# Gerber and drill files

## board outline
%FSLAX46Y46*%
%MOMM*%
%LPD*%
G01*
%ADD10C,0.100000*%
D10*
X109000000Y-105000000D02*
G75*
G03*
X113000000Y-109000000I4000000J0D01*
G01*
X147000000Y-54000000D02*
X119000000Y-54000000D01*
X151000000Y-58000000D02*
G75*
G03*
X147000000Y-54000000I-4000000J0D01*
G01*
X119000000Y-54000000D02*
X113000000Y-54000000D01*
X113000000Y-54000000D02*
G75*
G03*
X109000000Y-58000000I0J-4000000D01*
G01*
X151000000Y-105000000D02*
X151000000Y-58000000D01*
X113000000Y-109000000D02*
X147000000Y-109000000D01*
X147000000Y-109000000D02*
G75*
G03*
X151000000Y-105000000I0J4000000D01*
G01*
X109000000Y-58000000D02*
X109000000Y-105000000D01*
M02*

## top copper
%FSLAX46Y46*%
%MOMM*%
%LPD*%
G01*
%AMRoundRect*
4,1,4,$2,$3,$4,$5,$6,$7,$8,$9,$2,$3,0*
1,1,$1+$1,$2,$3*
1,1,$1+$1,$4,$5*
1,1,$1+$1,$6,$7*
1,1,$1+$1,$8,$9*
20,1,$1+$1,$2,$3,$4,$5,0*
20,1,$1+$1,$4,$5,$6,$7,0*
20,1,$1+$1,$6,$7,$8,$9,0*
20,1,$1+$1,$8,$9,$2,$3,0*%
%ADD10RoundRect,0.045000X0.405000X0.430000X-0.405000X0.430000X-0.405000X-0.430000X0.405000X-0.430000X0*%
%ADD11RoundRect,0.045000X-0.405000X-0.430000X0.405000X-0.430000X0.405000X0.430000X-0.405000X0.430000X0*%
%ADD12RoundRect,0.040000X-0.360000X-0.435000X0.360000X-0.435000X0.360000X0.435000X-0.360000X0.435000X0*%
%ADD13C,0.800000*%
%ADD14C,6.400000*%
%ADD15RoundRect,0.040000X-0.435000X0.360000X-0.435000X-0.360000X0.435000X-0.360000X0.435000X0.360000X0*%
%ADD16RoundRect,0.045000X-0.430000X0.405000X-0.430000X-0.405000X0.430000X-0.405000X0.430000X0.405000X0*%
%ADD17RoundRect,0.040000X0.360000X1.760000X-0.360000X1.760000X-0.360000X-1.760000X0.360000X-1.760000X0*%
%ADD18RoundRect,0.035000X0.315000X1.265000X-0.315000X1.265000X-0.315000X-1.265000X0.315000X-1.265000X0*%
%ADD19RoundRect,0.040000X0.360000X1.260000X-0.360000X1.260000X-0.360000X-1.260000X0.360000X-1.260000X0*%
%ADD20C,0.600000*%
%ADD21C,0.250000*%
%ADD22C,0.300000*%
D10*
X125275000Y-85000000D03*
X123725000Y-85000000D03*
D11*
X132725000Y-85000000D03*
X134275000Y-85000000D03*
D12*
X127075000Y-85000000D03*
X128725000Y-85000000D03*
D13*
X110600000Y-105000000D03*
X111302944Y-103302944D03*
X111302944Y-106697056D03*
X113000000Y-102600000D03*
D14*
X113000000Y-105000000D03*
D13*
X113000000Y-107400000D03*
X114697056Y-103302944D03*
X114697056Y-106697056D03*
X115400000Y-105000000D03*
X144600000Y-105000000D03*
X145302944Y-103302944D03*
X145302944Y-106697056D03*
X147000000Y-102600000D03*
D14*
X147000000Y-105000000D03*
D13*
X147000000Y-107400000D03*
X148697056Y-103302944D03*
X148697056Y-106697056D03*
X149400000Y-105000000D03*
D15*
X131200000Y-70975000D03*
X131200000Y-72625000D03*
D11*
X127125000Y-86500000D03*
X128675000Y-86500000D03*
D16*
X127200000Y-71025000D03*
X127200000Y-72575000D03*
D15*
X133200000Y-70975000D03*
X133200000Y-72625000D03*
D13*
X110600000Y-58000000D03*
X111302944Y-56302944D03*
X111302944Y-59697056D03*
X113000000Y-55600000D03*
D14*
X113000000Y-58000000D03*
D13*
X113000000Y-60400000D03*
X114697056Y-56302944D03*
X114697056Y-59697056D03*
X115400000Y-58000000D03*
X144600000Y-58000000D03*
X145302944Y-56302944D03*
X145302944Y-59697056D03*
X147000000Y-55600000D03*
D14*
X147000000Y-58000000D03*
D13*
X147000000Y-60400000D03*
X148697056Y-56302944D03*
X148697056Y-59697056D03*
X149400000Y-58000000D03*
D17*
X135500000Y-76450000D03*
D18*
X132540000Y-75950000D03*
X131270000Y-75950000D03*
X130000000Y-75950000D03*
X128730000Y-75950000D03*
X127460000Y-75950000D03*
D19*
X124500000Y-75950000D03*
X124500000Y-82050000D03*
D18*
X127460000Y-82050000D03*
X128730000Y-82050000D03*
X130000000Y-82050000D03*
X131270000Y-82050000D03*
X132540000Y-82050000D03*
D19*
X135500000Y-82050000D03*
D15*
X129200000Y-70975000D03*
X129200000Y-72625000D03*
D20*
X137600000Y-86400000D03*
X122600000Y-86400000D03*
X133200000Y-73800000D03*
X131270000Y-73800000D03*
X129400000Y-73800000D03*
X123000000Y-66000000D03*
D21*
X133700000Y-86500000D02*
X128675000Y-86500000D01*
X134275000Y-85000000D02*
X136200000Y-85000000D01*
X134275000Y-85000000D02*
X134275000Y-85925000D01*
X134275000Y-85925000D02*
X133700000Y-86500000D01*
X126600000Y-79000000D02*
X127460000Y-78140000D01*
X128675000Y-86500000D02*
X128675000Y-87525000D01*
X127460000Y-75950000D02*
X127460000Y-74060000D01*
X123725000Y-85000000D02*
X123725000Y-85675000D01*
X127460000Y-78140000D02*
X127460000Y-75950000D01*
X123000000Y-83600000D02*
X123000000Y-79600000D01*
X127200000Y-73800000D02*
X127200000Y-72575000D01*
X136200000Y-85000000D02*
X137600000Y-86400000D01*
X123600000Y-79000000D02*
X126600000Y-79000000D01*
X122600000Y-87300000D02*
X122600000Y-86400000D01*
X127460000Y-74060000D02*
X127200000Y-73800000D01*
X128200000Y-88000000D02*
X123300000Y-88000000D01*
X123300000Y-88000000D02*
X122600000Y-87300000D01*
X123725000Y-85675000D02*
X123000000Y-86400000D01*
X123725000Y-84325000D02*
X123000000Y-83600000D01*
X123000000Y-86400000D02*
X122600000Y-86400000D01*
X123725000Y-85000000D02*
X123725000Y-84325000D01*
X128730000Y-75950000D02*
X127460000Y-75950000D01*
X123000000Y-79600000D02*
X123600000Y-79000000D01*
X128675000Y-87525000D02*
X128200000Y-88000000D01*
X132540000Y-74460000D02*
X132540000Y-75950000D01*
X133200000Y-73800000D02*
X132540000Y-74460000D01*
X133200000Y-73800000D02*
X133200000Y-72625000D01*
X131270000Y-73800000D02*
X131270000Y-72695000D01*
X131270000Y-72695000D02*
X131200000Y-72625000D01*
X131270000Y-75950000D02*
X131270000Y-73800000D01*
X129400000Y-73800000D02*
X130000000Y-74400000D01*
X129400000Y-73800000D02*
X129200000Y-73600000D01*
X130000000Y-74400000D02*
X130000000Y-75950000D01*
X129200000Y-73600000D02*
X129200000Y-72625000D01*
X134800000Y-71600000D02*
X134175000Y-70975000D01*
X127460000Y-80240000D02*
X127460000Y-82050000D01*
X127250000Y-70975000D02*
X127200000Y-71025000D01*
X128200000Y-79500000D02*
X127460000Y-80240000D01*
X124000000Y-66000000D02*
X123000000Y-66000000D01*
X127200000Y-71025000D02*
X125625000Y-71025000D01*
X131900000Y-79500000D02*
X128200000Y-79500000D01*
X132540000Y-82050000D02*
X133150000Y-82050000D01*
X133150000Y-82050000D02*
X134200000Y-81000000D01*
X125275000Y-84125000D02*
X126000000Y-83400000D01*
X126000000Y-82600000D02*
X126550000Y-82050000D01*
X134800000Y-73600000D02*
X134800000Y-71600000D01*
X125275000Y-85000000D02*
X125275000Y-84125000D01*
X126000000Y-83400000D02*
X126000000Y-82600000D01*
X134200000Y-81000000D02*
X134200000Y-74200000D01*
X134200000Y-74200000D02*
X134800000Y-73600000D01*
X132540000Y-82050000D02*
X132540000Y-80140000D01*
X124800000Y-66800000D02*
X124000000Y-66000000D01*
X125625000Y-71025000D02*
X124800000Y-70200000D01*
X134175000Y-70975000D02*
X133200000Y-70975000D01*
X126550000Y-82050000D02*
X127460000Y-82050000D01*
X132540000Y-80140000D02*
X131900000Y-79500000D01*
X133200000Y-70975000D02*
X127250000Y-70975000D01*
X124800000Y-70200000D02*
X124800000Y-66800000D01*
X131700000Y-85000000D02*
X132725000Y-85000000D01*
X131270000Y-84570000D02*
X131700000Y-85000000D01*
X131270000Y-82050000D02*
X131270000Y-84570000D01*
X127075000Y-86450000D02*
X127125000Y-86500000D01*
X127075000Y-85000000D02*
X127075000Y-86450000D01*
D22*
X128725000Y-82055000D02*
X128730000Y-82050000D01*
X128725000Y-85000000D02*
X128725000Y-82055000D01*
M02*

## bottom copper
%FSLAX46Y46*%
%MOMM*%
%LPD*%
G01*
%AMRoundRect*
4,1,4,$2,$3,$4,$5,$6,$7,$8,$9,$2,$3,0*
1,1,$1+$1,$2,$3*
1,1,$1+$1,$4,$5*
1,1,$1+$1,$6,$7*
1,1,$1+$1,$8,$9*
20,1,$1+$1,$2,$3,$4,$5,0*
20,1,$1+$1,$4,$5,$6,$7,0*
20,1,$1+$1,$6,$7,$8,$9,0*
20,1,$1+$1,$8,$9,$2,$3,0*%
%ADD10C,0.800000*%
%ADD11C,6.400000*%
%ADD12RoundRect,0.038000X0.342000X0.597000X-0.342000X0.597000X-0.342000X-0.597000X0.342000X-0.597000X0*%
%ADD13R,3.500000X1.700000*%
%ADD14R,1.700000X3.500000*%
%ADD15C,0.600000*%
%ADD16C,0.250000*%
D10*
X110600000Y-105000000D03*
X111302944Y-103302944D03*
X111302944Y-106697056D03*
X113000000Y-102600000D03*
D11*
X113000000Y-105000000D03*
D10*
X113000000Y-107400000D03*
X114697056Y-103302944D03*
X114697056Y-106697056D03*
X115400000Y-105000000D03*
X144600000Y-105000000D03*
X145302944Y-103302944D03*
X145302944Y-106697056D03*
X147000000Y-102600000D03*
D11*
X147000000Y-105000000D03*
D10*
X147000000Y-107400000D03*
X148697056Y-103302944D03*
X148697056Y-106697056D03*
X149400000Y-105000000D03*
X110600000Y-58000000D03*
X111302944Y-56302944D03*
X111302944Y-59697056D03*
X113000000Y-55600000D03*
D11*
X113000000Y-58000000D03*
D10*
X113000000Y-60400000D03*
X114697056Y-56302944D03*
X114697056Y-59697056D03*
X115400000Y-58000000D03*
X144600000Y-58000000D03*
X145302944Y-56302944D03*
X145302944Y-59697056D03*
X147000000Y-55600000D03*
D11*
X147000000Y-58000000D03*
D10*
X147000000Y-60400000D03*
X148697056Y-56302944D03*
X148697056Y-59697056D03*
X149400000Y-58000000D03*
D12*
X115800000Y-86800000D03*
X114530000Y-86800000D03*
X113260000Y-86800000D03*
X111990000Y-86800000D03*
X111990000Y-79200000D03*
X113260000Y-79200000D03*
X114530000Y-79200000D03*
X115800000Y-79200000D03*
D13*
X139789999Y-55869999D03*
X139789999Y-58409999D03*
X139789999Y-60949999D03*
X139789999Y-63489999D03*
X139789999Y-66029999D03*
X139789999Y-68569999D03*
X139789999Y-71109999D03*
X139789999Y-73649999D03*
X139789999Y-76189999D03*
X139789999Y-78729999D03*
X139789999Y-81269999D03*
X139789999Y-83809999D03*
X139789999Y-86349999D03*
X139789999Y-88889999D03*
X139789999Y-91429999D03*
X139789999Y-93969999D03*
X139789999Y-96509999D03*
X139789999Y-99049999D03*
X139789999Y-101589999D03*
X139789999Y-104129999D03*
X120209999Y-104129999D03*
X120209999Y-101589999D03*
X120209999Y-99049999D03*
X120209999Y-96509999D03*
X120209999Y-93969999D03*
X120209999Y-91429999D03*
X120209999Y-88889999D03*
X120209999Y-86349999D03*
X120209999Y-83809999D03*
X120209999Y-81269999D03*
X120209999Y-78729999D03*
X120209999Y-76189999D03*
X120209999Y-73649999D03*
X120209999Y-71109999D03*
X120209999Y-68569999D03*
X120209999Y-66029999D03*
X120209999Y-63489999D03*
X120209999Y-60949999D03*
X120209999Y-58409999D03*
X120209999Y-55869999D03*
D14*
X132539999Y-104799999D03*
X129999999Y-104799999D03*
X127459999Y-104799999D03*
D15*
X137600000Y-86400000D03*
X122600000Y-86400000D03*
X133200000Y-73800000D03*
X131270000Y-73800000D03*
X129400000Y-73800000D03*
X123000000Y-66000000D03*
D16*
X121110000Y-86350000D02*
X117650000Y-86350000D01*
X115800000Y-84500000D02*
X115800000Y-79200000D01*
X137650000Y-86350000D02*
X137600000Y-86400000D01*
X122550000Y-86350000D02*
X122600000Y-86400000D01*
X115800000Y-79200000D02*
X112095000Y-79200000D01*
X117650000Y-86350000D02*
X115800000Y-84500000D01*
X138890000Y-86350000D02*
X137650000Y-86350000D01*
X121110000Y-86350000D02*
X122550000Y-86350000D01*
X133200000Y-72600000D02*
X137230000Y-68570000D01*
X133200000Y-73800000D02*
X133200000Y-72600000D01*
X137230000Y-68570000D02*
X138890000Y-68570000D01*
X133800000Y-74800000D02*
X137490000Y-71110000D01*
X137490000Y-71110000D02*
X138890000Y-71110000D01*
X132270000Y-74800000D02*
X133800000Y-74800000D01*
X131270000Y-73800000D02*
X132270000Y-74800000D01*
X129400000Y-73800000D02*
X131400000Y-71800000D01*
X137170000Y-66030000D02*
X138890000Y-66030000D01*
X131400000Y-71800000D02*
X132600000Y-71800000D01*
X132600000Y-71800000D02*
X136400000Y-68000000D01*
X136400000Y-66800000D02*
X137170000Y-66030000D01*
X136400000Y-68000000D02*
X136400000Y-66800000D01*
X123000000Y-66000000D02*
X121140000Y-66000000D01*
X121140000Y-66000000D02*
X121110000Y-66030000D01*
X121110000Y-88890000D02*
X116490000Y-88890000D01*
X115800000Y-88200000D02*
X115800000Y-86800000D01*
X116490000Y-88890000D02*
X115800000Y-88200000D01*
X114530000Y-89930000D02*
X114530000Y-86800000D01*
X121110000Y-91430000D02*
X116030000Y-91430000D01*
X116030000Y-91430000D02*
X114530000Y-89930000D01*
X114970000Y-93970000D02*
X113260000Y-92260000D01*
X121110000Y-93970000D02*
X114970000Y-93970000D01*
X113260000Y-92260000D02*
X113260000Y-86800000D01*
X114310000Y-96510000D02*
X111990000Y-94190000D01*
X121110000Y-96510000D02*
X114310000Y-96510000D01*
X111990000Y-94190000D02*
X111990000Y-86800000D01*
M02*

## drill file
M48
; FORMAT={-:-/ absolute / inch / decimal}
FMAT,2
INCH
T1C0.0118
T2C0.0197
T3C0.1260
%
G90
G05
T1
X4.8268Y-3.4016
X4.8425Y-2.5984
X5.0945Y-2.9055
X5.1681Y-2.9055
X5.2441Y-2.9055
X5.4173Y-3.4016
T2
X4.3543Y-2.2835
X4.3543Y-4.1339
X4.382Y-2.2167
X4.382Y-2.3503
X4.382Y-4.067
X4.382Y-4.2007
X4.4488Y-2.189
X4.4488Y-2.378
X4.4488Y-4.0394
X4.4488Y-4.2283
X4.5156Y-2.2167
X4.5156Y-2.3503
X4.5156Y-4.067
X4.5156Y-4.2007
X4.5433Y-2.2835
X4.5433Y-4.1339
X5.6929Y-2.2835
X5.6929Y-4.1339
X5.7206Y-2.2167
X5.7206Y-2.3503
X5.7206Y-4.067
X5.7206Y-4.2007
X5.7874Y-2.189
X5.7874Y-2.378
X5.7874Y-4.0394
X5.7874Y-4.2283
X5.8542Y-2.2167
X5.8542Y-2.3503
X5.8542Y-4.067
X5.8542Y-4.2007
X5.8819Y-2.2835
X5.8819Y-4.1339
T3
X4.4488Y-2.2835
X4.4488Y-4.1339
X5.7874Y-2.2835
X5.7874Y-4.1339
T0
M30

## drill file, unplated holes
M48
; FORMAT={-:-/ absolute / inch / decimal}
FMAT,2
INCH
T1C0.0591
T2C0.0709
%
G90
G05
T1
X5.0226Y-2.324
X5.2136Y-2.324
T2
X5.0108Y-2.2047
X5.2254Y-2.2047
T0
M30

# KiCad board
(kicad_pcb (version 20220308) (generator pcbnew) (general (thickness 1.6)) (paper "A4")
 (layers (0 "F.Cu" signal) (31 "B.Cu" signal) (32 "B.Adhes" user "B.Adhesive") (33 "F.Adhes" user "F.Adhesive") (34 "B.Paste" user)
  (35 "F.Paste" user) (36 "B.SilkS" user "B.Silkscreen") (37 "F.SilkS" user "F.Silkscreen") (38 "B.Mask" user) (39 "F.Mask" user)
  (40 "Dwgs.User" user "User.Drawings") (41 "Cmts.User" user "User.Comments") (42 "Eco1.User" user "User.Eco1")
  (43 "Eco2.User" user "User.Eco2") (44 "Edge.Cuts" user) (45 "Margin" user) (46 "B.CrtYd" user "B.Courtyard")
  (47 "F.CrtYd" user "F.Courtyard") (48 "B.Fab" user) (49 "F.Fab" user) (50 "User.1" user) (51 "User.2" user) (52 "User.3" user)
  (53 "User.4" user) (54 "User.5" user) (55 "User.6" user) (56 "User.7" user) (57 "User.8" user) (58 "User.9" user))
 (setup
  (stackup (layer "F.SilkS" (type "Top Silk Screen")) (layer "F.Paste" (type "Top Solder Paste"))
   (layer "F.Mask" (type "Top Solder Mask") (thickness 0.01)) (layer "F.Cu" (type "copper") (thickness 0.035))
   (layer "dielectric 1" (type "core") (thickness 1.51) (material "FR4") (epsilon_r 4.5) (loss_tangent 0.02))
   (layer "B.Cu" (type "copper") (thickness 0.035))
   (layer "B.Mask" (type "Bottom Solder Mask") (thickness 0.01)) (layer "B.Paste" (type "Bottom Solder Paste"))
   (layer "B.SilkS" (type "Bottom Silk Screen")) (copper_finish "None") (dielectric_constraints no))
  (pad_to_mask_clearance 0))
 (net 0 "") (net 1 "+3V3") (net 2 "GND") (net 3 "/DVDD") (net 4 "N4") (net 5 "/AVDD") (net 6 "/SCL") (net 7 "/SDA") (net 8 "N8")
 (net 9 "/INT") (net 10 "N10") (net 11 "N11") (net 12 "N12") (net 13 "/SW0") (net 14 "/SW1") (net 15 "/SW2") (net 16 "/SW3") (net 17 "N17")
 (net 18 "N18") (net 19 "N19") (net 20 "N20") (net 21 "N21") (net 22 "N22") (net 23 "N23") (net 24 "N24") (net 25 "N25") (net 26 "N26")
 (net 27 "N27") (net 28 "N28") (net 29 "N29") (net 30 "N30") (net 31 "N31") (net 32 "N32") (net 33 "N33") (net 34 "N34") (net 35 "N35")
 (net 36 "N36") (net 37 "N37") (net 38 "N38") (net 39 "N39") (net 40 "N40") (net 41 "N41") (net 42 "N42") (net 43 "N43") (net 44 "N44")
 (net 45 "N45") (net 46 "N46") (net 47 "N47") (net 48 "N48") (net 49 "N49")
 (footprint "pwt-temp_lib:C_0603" (layer "F.Cu") (at 124.5 85 180)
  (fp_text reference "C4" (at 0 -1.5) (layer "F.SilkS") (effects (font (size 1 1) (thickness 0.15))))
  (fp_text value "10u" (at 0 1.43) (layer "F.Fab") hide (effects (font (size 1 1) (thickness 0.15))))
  (pad "1" smd roundrect (at -0.775 0 180) (size 0.9 0.95) (layers "F.Cu" "F.Paste" "F.Mask") (roundrect_rratio 0.05) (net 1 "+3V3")
   (solder_mask_margin 0.1) (solder_paste_margin -0.1) (clearance 0.1))
  (pad "2" smd roundrect (at 0.775 0 180) (size 0.9 0.95) (layers "F.Cu" "F.Paste" "F.Mask") (roundrect_rratio 0.05) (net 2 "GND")
   (solder_mask_margin 0.1) (solder_paste_margin -0.1) (clearance 0.1)))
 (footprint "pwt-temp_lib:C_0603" (layer "F.Cu") (at 133.5 85)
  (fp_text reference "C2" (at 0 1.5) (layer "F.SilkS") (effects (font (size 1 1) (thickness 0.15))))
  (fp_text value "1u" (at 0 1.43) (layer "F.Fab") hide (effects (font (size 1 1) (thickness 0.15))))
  (pad "1" smd roundrect (at -0.775 0) (size 0.9 0.95) (layers "F.Cu" "F.Paste" "F.Mask") (roundrect_rratio 0.05) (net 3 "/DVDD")
   (solder_mask_margin 0.1) (solder_paste_margin -0.1) (clearance 0.1))
  (pad "2" smd roundrect (at 0.775 0) (size 0.9 0.95) (layers "F.Cu" "F.Paste" "F.Mask") (roundrect_rratio 0.05) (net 2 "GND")
   (solder_mask_margin 0.1) (solder_paste_margin -0.1) (clearance 0.1)))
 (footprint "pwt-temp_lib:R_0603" (layer "F.Cu") (at 127.9 85)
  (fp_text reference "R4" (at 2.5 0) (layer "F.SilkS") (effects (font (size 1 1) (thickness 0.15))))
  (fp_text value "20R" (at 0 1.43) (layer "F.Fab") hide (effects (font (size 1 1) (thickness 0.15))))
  (pad "1" smd roundrect (at -0.825 0) (size 0.8 0.95) (layers "F.Cu" "F.Paste" "F.Mask") (roundrect_rratio 0.05) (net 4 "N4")
   (solder_mask_margin 0.1) (solder_paste_margin -0.1) (clearance 0.1))
  (pad "2" smd roundrect (at 0.825 0) (size 0.8 0.95) (layers "F.Cu" "F.Paste" "F.Mask") (roundrect_rratio 0.05) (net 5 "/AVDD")
   (solder_mask_margin 0.1) (solder_paste_margin -0.1) (clearance 0.1)))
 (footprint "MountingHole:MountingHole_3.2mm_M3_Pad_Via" (layer "F.Cu") (at 113 105)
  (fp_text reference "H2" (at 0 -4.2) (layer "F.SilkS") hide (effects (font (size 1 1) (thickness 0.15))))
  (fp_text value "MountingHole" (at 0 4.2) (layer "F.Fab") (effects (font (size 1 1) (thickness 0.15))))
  (pad "1" thru_hole circle (at -2.4 0) (size 0.8 0.8) (drill 0.5) (layers *.Cu *.Mask))
  (pad "1" thru_hole circle (at -1.697056 -1.697056) (size 0.8 0.8) (drill 0.5) (layers *.Cu *.Mask))
  (pad "1" thru_hole circle (at -1.697056 1.697056) (size 0.8 0.8) (drill 0.5) (layers *.Cu *.Mask))
  (pad "1" thru_hole circle (at 0 -2.4) (size 0.8 0.8) (drill 0.5) (layers *.Cu *.Mask))
  (pad "1" thru_hole circle (at 0 0) (size 6.4 6.4) (drill 3.2) (layers *.Cu *.Mask))
  (pad "1" thru_hole circle (at 0 2.4) (size 0.8 0.8) (drill 0.5) (layers *.Cu *.Mask))
  (pad "1" thru_hole circle (at 1.697056 -1.697056) (size 0.8 0.8) (drill 0.5) (layers *.Cu *.Mask))
  (pad "1" thru_hole circle (at 1.697056 1.697056) (size 0.8 0.8) (drill 0.5) (layers *.Cu *.Mask))
  (pad "1" thru_hole circle (at 2.4 0) (size 0.8 0.8) (drill 0.5) (layers *.Cu *.Mask)))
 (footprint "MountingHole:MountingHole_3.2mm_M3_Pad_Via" (layer "F.Cu") (at 147 105)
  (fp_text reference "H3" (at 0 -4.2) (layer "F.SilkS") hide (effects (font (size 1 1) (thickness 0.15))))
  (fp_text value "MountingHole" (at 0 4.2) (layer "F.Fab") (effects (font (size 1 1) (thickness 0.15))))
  (pad "1" thru_hole circle (at -2.4 0) (size 0.8 0.8) (drill 0.5) (layers *.Cu *.Mask))
  (pad "1" thru_hole circle (at -1.697056 -1.697056) (size 0.8 0.8) (drill 0.5) (layers *.Cu *.Mask))
  (pad "1" thru_hole circle (at -1.697056 1.697056) (size 0.8 0.8) (drill 0.5) (layers *.Cu *.Mask))
  (pad "1" thru_hole circle (at 0 -2.4) (size 0.8 0.8) (drill 0.5) (layers *.Cu *.Mask))
  (pad "1" thru_hole circle (at 0 0) (size 6.4 6.4) (drill 3.2) (layers *.Cu *.Mask))
  (pad "1" thru_hole circle (at 0 2.4) (size 0.8 0.8) (drill 0.5) (layers *.Cu *.Mask))
  (pad "1" thru_hole circle (at 1.697056 -1.697056) (size 0.8 0.8) (drill 0.5) (layers *.Cu *.Mask))
  (pad "1" thru_hole circle (at 1.697056 1.697056) (size 0.8 0.8) (drill 0.5) (layers *.Cu *.Mask))
  (pad "1" thru_hole circle (at 2.4 0) (size 0.8 0.8) (drill 0.5) (layers *.Cu *.Mask)))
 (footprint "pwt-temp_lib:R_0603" (layer "F.Cu") (at 131.2 71.8 -90)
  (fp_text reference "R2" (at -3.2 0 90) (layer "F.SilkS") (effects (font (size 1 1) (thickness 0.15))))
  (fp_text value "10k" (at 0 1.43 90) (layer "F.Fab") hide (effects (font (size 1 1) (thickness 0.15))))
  (pad "1" smd roundrect (at -0.825 0 270) (size 0.8 0.95) (layers "F.Cu" "F.Paste" "F.Mask") (roundrect_rratio 0.05) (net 1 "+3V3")
   (solder_mask_margin 0.1) (solder_paste_margin -0.1) (clearance 0.1))
  (pad "2" smd roundrect (at 0.825 0 270) (size 0.8 0.95) (layers "F.Cu" "F.Paste" "F.Mask") (roundrect_rratio 0.05) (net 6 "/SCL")
   (solder_mask_margin 0.1) (solder_paste_margin -0.1) (clearance 0.1)))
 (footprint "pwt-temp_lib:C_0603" (layer "F.Cu") (at 127.9 86.5)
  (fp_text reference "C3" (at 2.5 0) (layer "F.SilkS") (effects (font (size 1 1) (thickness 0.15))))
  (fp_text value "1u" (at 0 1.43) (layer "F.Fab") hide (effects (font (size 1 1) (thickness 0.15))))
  (pad "1" smd roundrect (at -0.775 0) (size 0.9 0.95) (layers "F.Cu" "F.Paste" "F.Mask") (roundrect_rratio 0.05) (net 4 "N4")
   (solder_mask_margin 0.1) (solder_paste_margin -0.1) (clearance 0.1))
  (pad "2" smd roundrect (at 0.775 0) (size 0.9 0.95) (layers "F.Cu" "F.Paste" "F.Mask") (roundrect_rratio 0.05) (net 2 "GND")
   (solder_mask_margin 0.1) (solder_paste_margin -0.1) (clearance 0.1)))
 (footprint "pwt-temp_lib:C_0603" (layer "F.Cu") (at 127.2 71.8 -90)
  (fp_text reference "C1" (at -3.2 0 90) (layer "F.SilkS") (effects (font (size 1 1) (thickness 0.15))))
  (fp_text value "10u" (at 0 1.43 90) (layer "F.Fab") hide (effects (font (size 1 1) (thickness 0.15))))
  (pad "1" smd roundrect (at -0.775 0 270) (size 0.9 0.95) (layers "F.Cu" "F.Paste" "F.Mask") (roundrect_rratio 0.05) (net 1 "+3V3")
   (solder_mask_margin 0.1) (solder_paste_margin -0.1) (clearance 0.1))
  (pad "2" smd roundrect (at 0.775 0 270) (size 0.9 0.95) (layers "F.Cu" "F.Paste" "F.Mask") (roundrect_rratio 0.05) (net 2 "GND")
   (solder_mask_margin 0.1) (solder_paste_margin -0.1) (clearance 0.1)))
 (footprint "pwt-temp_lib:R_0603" (layer "F.Cu") (at 133.2 71.8 -90)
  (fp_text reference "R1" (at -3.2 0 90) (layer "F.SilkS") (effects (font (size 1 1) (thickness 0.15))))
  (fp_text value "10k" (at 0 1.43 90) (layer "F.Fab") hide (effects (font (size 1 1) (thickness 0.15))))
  (pad "1" smd roundrect (at -0.825 0 270) (size 0.8 0.95) (layers "F.Cu" "F.Paste" "F.Mask") (roundrect_rratio 0.05) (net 1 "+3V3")
   (solder_mask_margin 0.1) (solder_paste_margin -0.1) (clearance 0.1))
  (pad "2" smd roundrect (at 0.825 0 270) (size 0.8 0.95) (layers "F.Cu" "F.Paste" "F.Mask") (roundrect_rratio 0.05) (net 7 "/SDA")
   (solder_mask_margin 0.1) (solder_paste_margin -0.1) (clearance 0.1)))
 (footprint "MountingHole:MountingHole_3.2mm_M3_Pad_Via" (layer "F.Cu") (at 113 58)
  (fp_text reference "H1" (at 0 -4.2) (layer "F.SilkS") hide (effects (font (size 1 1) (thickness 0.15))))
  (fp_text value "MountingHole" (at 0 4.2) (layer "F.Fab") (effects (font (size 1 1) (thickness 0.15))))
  (pad "1" thru_hole circle (at -2.4 0) (size 0.8 0.8) (drill 0.5) (layers *.Cu *.Mask))
  (pad "1" thru_hole circle (at -1.697056 -1.697056) (size 0.8 0.8) (drill 0.5) (layers *.Cu *.Mask))
  (pad "1" thru_hole circle (at -1.697056 1.697056) (size 0.8 0.8) (drill 0.5) (layers *.Cu *.Mask))
  (pad "1" thru_hole circle (at 0 -2.4) (size 0.8 0.8) (drill 0.5) (layers *.Cu *.Mask))
  (pad "1" thru_hole circle (at 0 0) (size 6.4 6.4) (drill 3.2) (layers *.Cu *.Mask))
  (pad "1" thru_hole circle (at 0 2.4) (size 0.8 0.8) (drill 0.5) (layers *.Cu *.Mask))
  (pad "1" thru_hole circle (at 1.697056 -1.697056) (size 0.8 0.8) (drill 0.5) (layers *.Cu *.Mask))
  (pad "1" thru_hole circle (at 1.697056 1.697056) (size 0.8 0.8) (drill 0.5) (layers *.Cu *.Mask))
  (pad "1" thru_hole circle (at 2.4 0) (size 0.8 0.8) (drill 0.5) (layers *.Cu *.Mask)))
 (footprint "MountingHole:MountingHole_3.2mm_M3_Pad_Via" (layer "F.Cu") (at 147 58)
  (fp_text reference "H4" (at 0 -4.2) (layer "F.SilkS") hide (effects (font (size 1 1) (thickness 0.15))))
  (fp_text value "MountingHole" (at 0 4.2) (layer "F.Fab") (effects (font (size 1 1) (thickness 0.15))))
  (pad "1" thru_hole circle (at -2.4 0) (size 0.8 0.8) (drill 0.5) (layers *.Cu *.Mask))
  (pad "1" thru_hole circle (at -1.697056 -1.697056) (size 0.8 0.8) (drill 0.5) (layers *.Cu *.Mask))
  (pad "1" thru_hole circle (at -1.697056 1.697056) (size 0.8 0.8) (drill 0.5) (layers *.Cu *.Mask))
  (pad "1" thru_hole circle (at 0 -2.4) (size 0.8 0.8) (drill 0.5) (layers *.Cu *.Mask))
  (pad "1" thru_hole circle (at 0 0) (size 6.4 6.4) (drill 3.2) (layers *.Cu *.Mask))
  (pad "1" thru_hole circle (at 0 2.4) (size 0.8 0.8) (drill 0.5) (layers *.Cu *.Mask))
  (pad "1" thru_hole circle (at 1.697056 -1.697056) (size 0.8 0.8) (drill 0.5) (layers *.Cu *.Mask))
  (pad "1" thru_hole circle (at 1.697056 1.697056) (size 0.8 0.8) (drill 0.5) (layers *.Cu *.Mask))
  (pad "1" thru_hole circle (at 2.4 0) (size 0.8 0.8) (drill 0.5) (layers *.Cu *.Mask)))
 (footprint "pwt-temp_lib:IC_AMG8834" (layer "F.Cu") (at 130 79 180)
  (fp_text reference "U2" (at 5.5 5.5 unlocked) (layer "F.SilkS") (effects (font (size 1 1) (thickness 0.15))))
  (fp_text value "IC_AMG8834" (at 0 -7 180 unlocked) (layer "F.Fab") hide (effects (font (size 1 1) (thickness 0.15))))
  (pad "1" smd roundrect (at -5.5 2.55 180) (size 0.8 3.6) (layers "F.Cu" "F.Paste" "F.Mask") (roundrect_rratio 0.05) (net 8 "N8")
   (solder_mask_margin 0.1) (solder_paste_margin -0.1) (clearance 0.2) (thermal_bridge_angle 45))
  (pad "2" smd roundrect (at -2.54 3.05 180) (size 0.7 2.6) (layers "F.Cu" "F.Paste" "F.Mask") (roundrect_rratio 0.05) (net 7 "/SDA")
   (solder_mask_margin 0.1) (solder_paste_margin -0.1) (clearance 0.2) (thermal_bridge_angle 45))
  (pad "3" smd roundrect (at -1.27 3.05 180) (size 0.7 2.6) (layers "F.Cu" "F.Paste" "F.Mask") (roundrect_rratio 0.05) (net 6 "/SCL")
   (solder_mask_margin 0.1) (solder_paste_margin -0.1) (clearance 0.2) (thermal_bridge_angle 45))
  (pad "4" smd roundrect (at 0 3.05 180) (size 0.7 2.6) (layers "F.Cu" "F.Paste" "F.Mask") (roundrect_rratio 0.05) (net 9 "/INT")
   (solder_mask_margin 0.1) (solder_paste_margin -0.1) (clearance 0.2) (thermal_bridge_angle 45))
  (pad "5" smd roundrect (at 1.27 3.05 180) (size 0.7 2.6) (layers "F.Cu" "F.Paste" "F.Mask") (roundrect_rratio 0.05) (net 2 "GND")
   (solder_mask_margin 0.1) (solder_paste_margin -0.1) (clearance 0.2) (thermal_bridge_angle 45))
  (pad "6" smd roundrect (at 2.54 3.05 180) (size 0.7 2.6) (layers "F.Cu" "F.Paste" "F.Mask") (roundrect_rratio 0.05) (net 2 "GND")
   (solder_mask_margin 0.1) (solder_paste_margin -0.1) (clearance 0.2) (thermal_bridge_angle 45))
  (pad "7" smd roundrect (at 5.5 3.05 180) (size 0.8 2.6) (layers "F.Cu" "F.Paste" "F.Mask") (roundrect_rratio 0.05) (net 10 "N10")
   (solder_mask_margin 0.1) (solder_paste_margin -0.1) (clearance 0.2) (thermal_bridge_angle 45))
  (pad "8" smd roundrect (at 5.5 -3.05 180) (size 0.8 2.6) (layers "F.Cu" "F.Paste" "F.Mask") (roundrect_rratio 0.05) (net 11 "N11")
   (solder_mask_margin 0.1) (solder_paste_margin -0.1) (clearance 0.2) (thermal_bridge_angle 45))
  (pad "9" smd roundrect (at 2.54 -3.05 180) (size 0.7 2.6) (layers "F.Cu" "F.Paste" "F.Mask") (roundrect_rratio 0.05) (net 1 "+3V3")
   (solder_mask_margin 0.1) (solder_paste_margin -0.1) (clearance 0.2) (thermal_bridge_angle 45))
  (pad "10" smd roundrect (at 1.27 -3.05 180) (size 0.7 2.6) (layers "F.Cu" "F.Paste" "F.Mask") (roundrect_rratio 0.05) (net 5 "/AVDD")
   (solder_mask_margin 0.1) (solder_paste_margin -0.1) (clearance 0.2) (thermal_bridge_angle 45))
  (pad "11" smd roundrect (at 0 -3.05 180) (size 0.7 2.6) (layers "F.Cu" "F.Paste" "F.Mask") (roundrect_rratio 0.05) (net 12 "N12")
   (solder_mask_margin 0.1) (solder_paste_margin -0.1) (clearance 0.2) (thermal_bridge_angle 45))
  (pad "12" smd roundrect (at -1.27 -3.05 180) (size 0.7 2.6) (layers "F.Cu" "F.Paste" "F.Mask") (roundrect_rratio 0.05) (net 3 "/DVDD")
   (solder_mask_margin 0.1) (solder_paste_margin -0.1) (clearance 0.2) (thermal_bridge_angle 45))
  (pad "13" smd roundrect (at -2.54 -3.05 180) (size 0.7 2.6) (layers "F.Cu" "F.Paste" "F.Mask") (roundrect_rratio 0.05) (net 1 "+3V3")
   (solder_mask_margin 0.1) (solder_paste_margin -0.1) (clearance 0.2) (thermal_bridge_angle 45))
  (pad "14" smd roundrect (at -5.5 -3.05 180) (size 0.8 2.6) (layers "F.Cu" "F.Paste" "F.Mask") (roundrect_rratio 0.05)
   (solder_mask_margin 0.1) (solder_paste_margin -0.1) (clearance 0.2) (thermal_bridge_angle 45)))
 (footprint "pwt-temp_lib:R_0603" (layer "F.Cu") (at 129.2 71.8 -90)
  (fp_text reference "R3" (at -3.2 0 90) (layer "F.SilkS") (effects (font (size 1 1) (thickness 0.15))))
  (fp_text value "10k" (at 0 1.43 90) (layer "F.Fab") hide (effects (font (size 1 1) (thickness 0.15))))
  (pad "1" smd roundrect (at -0.825 0 270) (size 0.8 0.95) (layers "F.Cu" "F.Paste" "F.Mask") (roundrect_rratio 0.05) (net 1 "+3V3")
   (solder_mask_margin 0.1) (solder_paste_margin -0.1) (clearance 0.1))
  (pad "2" smd roundrect (at 0.825 0 270) (size 0.8 0.95) (layers "F.Cu" "F.Paste" "F.Mask") (roundrect_rratio 0.05) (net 9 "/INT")
   (solder_mask_margin 0.1) (solder_paste_margin -0.1) (clearance 0.1)))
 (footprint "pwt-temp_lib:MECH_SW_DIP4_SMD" (layer "B.Cu") (at 113.895 83 180)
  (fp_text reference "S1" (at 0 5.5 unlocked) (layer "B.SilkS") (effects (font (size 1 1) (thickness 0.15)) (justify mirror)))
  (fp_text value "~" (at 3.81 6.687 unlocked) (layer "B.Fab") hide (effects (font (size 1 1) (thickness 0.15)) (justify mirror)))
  (pad "1" smd roundrect (at -1.905 -3.8 180) (size 0.76 1.27) (layers "B.Cu" "B.Paste" "B.Mask") (roundrect_rratio 0.05) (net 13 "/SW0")
   (solder_mask_margin 0.1) (solder_paste_margin -0.1) (clearance 0.1) (thermal_bridge_angle 45))
  (pad "2" smd roundrect (at -0.635 -3.8 180) (size 0.76 1.27) (layers "B.Cu" "B.Paste" "B.Mask") (roundrect_rratio 0.05) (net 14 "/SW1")
   (solder_mask_margin 0.1) (solder_paste_margin -0.1) (clearance 0.1) (thermal_bridge_angle 45))
  (pad "3" smd roundrect (at 0.635 -3.8 180) (size 0.76 1.27) (layers "B.Cu" "B.Paste" "B.Mask") (roundrect_rratio 0.05) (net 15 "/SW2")
   (solder_mask_margin 0.1) (solder_paste_margin -0.1) (clearance 0.1) (thermal_bridge_angle 45))
  (pad "4" smd roundrect (at 1.905 -3.8 180) (size 0.76 1.27) (layers "B.Cu" "B.Paste" "B.Mask") (roundrect_rratio 0.05) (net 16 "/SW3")
   (solder_mask_margin 0.1) (solder_paste_margin -0.1) (clearance 0.1) (thermal_bridge_angle 45))
  (pad "5" smd roundrect (at 1.905 3.8 180) (size 0.76 1.27) (layers "B.Cu" "B.Paste" "B.Mask") (roundrect_rratio 0.05) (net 2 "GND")
   (solder_mask_margin 0.1) (solder_paste_margin -0.1) (clearance 0.1) (thermal_bridge_angle 45))
  (pad "6" smd roundrect (at 0.635 3.8 180) (size 0.76 1.27) (layers "B.Cu" "B.Paste" "B.Mask") (roundrect_rratio 0.05) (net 2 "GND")
   (solder_mask_margin 0.1) (solder_paste_margin -0.1) (clearance 0.1) (thermal_bridge_angle 45))
  (pad "7" smd roundrect (at -0.635 3.8 180) (size 0.76 1.27) (layers "B.Cu" "B.Paste" "B.Mask") (roundrect_rratio 0.05) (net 2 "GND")
   (solder_mask_margin 0.1) (solder_paste_margin -0.1) (clearance 0.1) (thermal_bridge_angle 45))
  (pad "8" smd roundrect (at -1.905 3.8 180) (size 0.76 1.27) (layers "B.Cu" "B.Paste" "B.Mask") (roundrect_rratio 0.05) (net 2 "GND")
   (solder_mask_margin 0.1) (solder_paste_margin -0.1) (clearance 0.1) (thermal_bridge_angle 45)))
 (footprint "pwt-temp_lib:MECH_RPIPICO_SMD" (layer "B.Cu") (at 130 80 180)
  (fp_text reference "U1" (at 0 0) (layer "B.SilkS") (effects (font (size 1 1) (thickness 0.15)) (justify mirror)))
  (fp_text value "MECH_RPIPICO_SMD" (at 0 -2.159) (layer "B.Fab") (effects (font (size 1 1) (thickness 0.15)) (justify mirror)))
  (pad "" np_thru_hole oval (at -2.725 24 180) (size 1.8 1.8) (drill 1.8) (layers *.Cu *.Mask))
  (pad "" np_thru_hole oval (at -2.425 20.97 180) (size 1.5 1.5) (drill 1.5) (layers *.Cu *.Mask))
  (pad "" np_thru_hole oval (at 2.425 20.97 180) (size 1.5 1.5) (drill 1.5) (layers *.Cu *.Mask))
  (pad "" np_thru_hole oval (at 2.725 24 180) (size 1.8 1.8) (drill 1.8) (layers *.Cu *.Mask))
  (pad "1" smd rect (at -8.89 24.13 180) (size 3.5 1.7) (drill (offset -0.9 0)) (layers "B.Cu" "B.Mask") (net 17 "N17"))
  (pad "2" smd rect (at -8.89 21.59 180) (size 3.5 1.7) (drill (offset -0.9 0)) (layers "B.Cu" "B.Mask") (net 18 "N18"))
  (pad "3" smd rect (at -8.89 19.05 180) (size 3.5 1.7) (drill (offset -0.9 0)) (layers "B.Cu" "B.Mask") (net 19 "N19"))
  (pad "4" smd rect (at -8.89 16.51 180) (size 3.5 1.7) (drill (offset -0.9 0)) (layers "B.Cu" "B.Mask") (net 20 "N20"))
  (pad "5" smd rect (at -8.89 13.97 180) (size 3.5 1.7) (drill (offset -0.9 0)) (layers "B.Cu" "B.Mask") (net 9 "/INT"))
  (pad "6" smd rect (at -8.89 11.43 180) (size 3.5 1.7) (drill (offset -0.9 0)) (layers "B.Cu" "B.Mask") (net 7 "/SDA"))
  (pad "7" smd rect (at -8.89 8.89 180) (size 3.5 1.7) (drill (offset -0.9 0)) (layers "B.Cu" "B.Mask") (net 6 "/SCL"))
  (pad "8" smd rect (at -8.89 6.35 180) (size 3.5 1.7) (drill (offset -0.9 0)) (layers "B.Cu" "B.Mask") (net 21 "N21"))
  (pad "9" smd rect (at -8.89 3.81 180) (size 3.5 1.7) (drill (offset -0.9 0)) (layers "B.Cu" "B.Mask") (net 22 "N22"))
  (pad "10" smd rect (at -8.89 1.27 180) (size 3.5 1.7) (drill (offset -0.9 0)) (layers "B.Cu" "B.Mask") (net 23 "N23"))
  (pad "11" smd rect (at -8.89 -1.27 180) (size 3.5 1.7) (drill (offset -0.9 0)) (layers "B.Cu" "B.Mask") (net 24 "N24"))
  (pad "12" smd rect (at -8.89 -3.81 180) (size 3.5 1.7) (drill (offset -0.9 0)) (layers "B.Cu" "B.Mask") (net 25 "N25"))
  (pad "13" smd rect (at -8.89 -6.35 180) (size 3.5 1.7) (drill (offset -0.9 0)) (layers "B.Cu" "B.Mask") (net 2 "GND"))
  (pad "14" smd rect (at -8.89 -8.89 180) (size 3.5 1.7) (drill (offset -0.9 0)) (layers "B.Cu" "B.Mask") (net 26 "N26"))
  (pad "15" smd rect (at -8.89 -11.43 180) (size 3.5 1.7) (drill (offset -0.9 0)) (layers "B.Cu" "B.Mask") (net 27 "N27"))
  (pad "16" smd rect (at -8.89 -13.97 180) (size 3.5 1.7) (drill (offset -0.9 0)) (layers "B.Cu" "B.Mask") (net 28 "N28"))
  (pad "17" smd rect (at -8.89 -16.51 180) (size 3.5 1.7) (drill (offset -0.9 0)) (layers "B.Cu" "B.Mask") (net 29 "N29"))
  (pad "18" smd rect (at -8.89 -19.05 180) (size 3.5 1.7) (drill (offset -0.9 0)) (layers "B.Cu" "B.Mask") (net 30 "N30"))
  (pad "19" smd rect (at -8.89 -21.59 180) (size 3.5 1.7) (drill (offset -0.9 0)) (layers "B.Cu" "B.Mask") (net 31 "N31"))
  (pad "20" smd rect (at -8.89 -24.13 180) (size 3.5 1.7) (drill (offset -0.9 0)) (layers "B.Cu" "B.Mask") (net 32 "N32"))
  (pad "21" smd rect (at 8.89 -24.13 180) (size 3.5 1.7) (drill (offset 0.9 0)) (layers "B.Cu" "B.Mask") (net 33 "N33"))
  (pad "22" smd rect (at 8.89 -21.59 180) (size 3.5 1.7) (drill (offset 0.9 0)) (layers "B.Cu" "B.Mask") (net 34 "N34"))
  (pad "23" smd rect (at 8.89 -19.05 180) (size 3.5 1.7) (drill (offset 0.9 0)) (layers "B.Cu" "B.Mask") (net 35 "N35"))
  (pad "24" smd rect (at 8.89 -16.51 180) (size 3.5 1.7) (drill (offset 0.9 0)) (layers "B.Cu" "B.Mask") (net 16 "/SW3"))
  (pad "25" smd rect (at 8.89 -13.97 180) (size 3.5 1.7) (drill (offset 0.9 0)) (layers "B.Cu" "B.Mask") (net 15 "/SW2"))
  (pad "26" smd rect (at 8.89 -11.43 180) (size 3.5 1.7) (drill (offset 0.9 0)) (layers "B.Cu" "B.Mask") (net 14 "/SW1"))
  (pad "27" smd rect (at 8.89 -8.89 180) (size 3.5 1.7) (drill (offset 0.9 0)) (layers "B.Cu" "B.Mask") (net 13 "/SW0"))
  (pad "28" smd rect (at 8.89 -6.35 180) (size 3.5 1.7) (drill (offset 0.9 0)) (layers "B.Cu" "B.Mask") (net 2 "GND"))
  (pad "29" smd rect (at 8.89 -3.81 180) (size 3.5 1.7) (drill (offset 0.9 0)) (layers "B.Cu" "B.Mask") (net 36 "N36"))
  (pad "30" smd rect (at 8.89 -1.27 180) (size 3.5 1.7) (drill (offset 0.9 0)) (layers "B.Cu" "B.Mask") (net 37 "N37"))
  (pad "31" smd rect (at 8.89 1.27 180) (size 3.5 1.7) (drill (offset 0.9 0)) (layers "B.Cu" "B.Mask") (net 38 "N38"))
  (pad "32" smd rect (at 8.89 3.81 180) (size 3.5 1.7) (drill (offset 0.9 0)) (layers "B.Cu" "B.Mask") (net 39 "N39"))
  (pad "33" smd rect (at 8.89 6.35 180) (size 3.5 1.7) (drill (offset 0.9 0)) (layers "B.Cu" "B.Mask") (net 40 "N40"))
  (pad "34" smd rect (at 8.89 8.89 180) (size 3.5 1.7) (drill (offset 0.9 0)) (layers "B.Cu" "B.Mask") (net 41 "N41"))
  (pad "35" smd rect (at 8.89 11.43 180) (size 3.5 1.7) (drill (offset 0.9 0)) (layers "B.Cu" "B.Mask") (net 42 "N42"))
  (pad "36" smd rect (at 8.89 13.97 180) (size 3.5 1.7) (drill (offset 0.9 0)) (layers "B.Cu" "B.Mask") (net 1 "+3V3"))
  (pad "37" smd rect (at 8.89 16.51 180) (size 3.5 1.7) (drill (offset 0.9 0)) (layers "B.Cu" "B.Mask") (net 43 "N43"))
  (pad "38" smd rect (at 8.89 19.05 180) (size 3.5 1.7) (drill (offset 0.9 0)) (layers "B.Cu" "B.Mask") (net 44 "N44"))
  (pad "39" smd rect (at 8.89 21.59 180) (size 3.5 1.7) (drill (offset 0.9 0)) (layers "B.Cu" "B.Mask") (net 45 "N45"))
  (pad "40" smd rect (at 8.89 24.13 180) (size 3.5 1.7) (drill (offset 0.9 0)) (layers "B.Cu" "B.Mask") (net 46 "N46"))
  (pad "41" smd rect (at -2.54 -23.9 90) (size 3.5 1.7) (drill (offset -0.9 0)) (layers "B.Cu" "B.Mask") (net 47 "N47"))
  (pad "42" smd rect (at 0 -23.9 90) (size 3.5 1.7) (drill (offset -0.9 0)) (layers "B.Cu" "B.Mask") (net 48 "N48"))
  (pad "43" smd rect (at 2.54 -23.9 90) (size 3.5 1.7) (drill (offset -0.9 0)) (layers "B.Cu" "B.Mask") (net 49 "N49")))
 (gr_arc (start 113 109) (mid 110.171573 107.828427) (end 109 105) (stroke (width 0.1) (type default)) (layer "Edge.Cuts"))
 (gr_line (start 147 54) (end 119 54) (stroke (width 0.1) (type default)) (layer "Edge.Cuts"))
 (gr_arc (start 147 54) (mid 149.828427 55.171573) (end 151 58) (stroke (width 0.1) (type default)) (layer "Edge.Cuts"))
 (gr_line (start 119 54) (end 113 54) (stroke (width 0.1) (type default)) (layer "Edge.Cuts"))
 (gr_arc (start 109 58) (mid 110.171573 55.171573) (end 113 54) (stroke (width 0.1) (type default)) (layer "Edge.Cuts"))
 (gr_line (start 151 105) (end 151 58) (stroke (width 0.1) (type default)) (layer "Edge.Cuts"))
 (gr_line (start 113 109) (end 147 109) (stroke (width 0.1) (type default)) (layer "Edge.Cuts"))
 (gr_arc (start 151 105) (mid 149.828427 107.828427) (end 147 109) (stroke (width 0.1) (type default)) (layer "Edge.Cuts"))
 (gr_line (start 109 58) (end 109 105) (stroke (width 0.1) (type default)) (layer "Edge.Cuts"))
 (segment (start 133.7 86.5) (end 128.675 86.5) (width 0.25) (layer "F.Cu") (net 2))
 (segment (start 134.275 85) (end 136.2 85) (width 0.25) (layer "F.Cu") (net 2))
 (segment (start 134.275 85) (end 134.275 85.925) (width 0.25) (layer "F.Cu") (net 2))
 (segment (start 134.275 85.925) (end 133.7 86.5) (width 0.25) (layer "F.Cu") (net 2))
 (segment (start 126.6 79) (end 127.46 78.14) (width 0.25) (layer "F.Cu") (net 2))
 (segment (start 128.675 86.5) (end 128.675 87.525) (width 0.25) (layer "F.Cu") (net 2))
 (segment (start 127.46 75.95) (end 127.46 74.06) (width 0.25) (layer "F.Cu") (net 2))
 (segment (start 123.725 85) (end 123.725 85.675) (width 0.25) (layer "F.Cu") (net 2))
 (segment (start 127.46 78.14) (end 127.46 75.95) (width 0.25) (layer "F.Cu") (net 2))
 (segment (start 123 83.6) (end 123 79.6) (width 0.25) (layer "F.Cu") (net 2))
 (segment (start 127.2 73.8) (end 127.2 72.575) (width 0.25) (layer "F.Cu") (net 2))
 (segment (start 136.2 85) (end 137.6 86.4) (width 0.25) (layer "F.Cu") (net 2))
 (segment (start 123.6 79) (end 126.6 79) (width 0.25) (layer "F.Cu") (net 2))
 (segment (start 122.6 87.3) (end 122.6 86.4) (width 0.25) (layer "F.Cu") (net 2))
 (segment (start 127.46 74.06) (end 127.2 73.8) (width 0.25) (layer "F.Cu") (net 2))
 (segment (start 128.2 88) (end 123.3 88) (width 0.25) (layer "F.Cu") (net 2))
 (segment (start 123.3 88) (end 122.6 87.3) (width 0.25) (layer "F.Cu") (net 2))
 (segment (start 123.725 85.675) (end 123 86.4) (width 0.25) (layer "F.Cu") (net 2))
 (segment (start 123.725 84.325) (end 123 83.6) (width 0.25) (layer "F.Cu") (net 2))
 (segment (start 123 86.4) (end 122.6 86.4) (width 0.25) (layer "F.Cu") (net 2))
 (segment (start 123.725 85) (end 123.725 84.325) (width 0.25) (layer "F.Cu") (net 2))
 (segment (start 128.73 75.95) (end 127.46 75.95) (width 0.25) (layer "F.Cu") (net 2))
 (segment (start 123 79.6) (end 123.6 79) (width 0.25) (layer "F.Cu") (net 2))
 (segment (start 128.675 87.525) (end 128.2 88) (width 0.25) (layer "F.Cu") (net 2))
 (via (at 137.6 86.4) (size 0.6) (drill 0.3) (layers "F.Cu" "B.Cu") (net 2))
 (via (at 122.6 86.4) (size 0.6) (drill 0.3) (layers "F.Cu" "B.Cu") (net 2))
 (segment (start 121.11 86.35) (end 117.65 86.35) (width 0.25) (layer "B.Cu") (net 2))
 (segment (start 115.8 84.5) (end 115.8 79.2) (width 0.25) (layer "B.Cu") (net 2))
 (segment (start 137.65 86.35) (end 137.6 86.4) (width 0.25) (layer "B.Cu") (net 2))
 (segment (start 122.55 86.35) (end 122.6 86.4) (width 0.25) (layer "B.Cu") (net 2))
 (segment (start 115.8 79.2) (end 112.095 79.2) (width 0.25) (layer "B.Cu") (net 2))
 (segment (start 117.65 86.35) (end 115.8 84.5) (width 0.25) (layer "B.Cu") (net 2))
 (segment (start 138.89 86.35) (end 137.65 86.35) (width 0.25) (layer "B.Cu") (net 2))
 (segment (start 121.11 86.35) (end 122.55 86.35) (width 0.25) (layer "B.Cu") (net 2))
 (segment (start 132.54 74.46) (end 132.54 75.95) (width 0.25) (layer "F.Cu") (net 7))
 (segment (start 133.2 73.8) (end 132.54 74.46) (width 0.25) (layer "F.Cu") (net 7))
 (segment (start 133.2 73.8) (end 133.2 72.625) (width 0.25) (layer "F.Cu") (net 7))
 (via (at 133.2 73.8) (size 0.6) (drill 0.3) (layers "F.Cu" "B.Cu") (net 7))
 (segment (start 133.2 72.6) (end 137.23 68.57) (width 0.25) (layer "B.Cu") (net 7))
 (segment (start 133.2 73.8) (end 133.2 72.6) (width 0.25) (layer "B.Cu") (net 7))
 (segment (start 137.23 68.57) (end 138.89 68.57) (width 0.25) (layer "B.Cu") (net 7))
 (segment (start 131.27 73.8) (end 131.27 72.695) (width 0.25) (layer "F.Cu") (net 6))
 (segment (start 131.27 72.695) (end 131.2 72.625) (width 0.25) (layer "F.Cu") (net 6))
 (segment (start 131.27 75.95) (end 131.27 73.8) (width 0.25) (layer "F.Cu") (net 6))
 (via (at 131.27 73.8) (size 0.6) (drill 0.3) (layers "F.Cu" "B.Cu") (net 6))
 (segment (start 133.8 74.8) (end 137.49 71.11) (width 0.25) (layer "B.Cu") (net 6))
 (segment (start 137.49 71.11) (end 138.89 71.11) (width 0.25) (layer "B.Cu") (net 6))
 (segment (start 132.27 74.8) (end 133.8 74.8) (width 0.25) (layer "B.Cu") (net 6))
 (segment (start 131.27 73.8) (end 132.27 74.8) (width 0.25) (layer "B.Cu") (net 6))
 (segment (start 129.4 73.8) (end 130 74.4) (width 0.25) (layer "F.Cu") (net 9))
 (segment (start 129.4 73.8) (end 129.2 73.6) (width 0.25) (layer "F.Cu") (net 9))
 (segment (start 130 74.4) (end 130 75.95) (width 0.25) (layer "F.Cu") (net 9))
 (segment (start 129.2 73.6) (end 129.2 72.625) (width 0.25) (layer "F.Cu") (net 9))
 (via (at 129.4 73.8) (size 0.6) (drill 0.3) (layers "F.Cu" "B.Cu") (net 9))
 (segment (start 129.4 73.8) (end 131.4 71.8) (width 0.25) (layer "B.Cu") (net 9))
 (segment (start 137.17 66.03) (end 138.89 66.03) (width 0.25) (layer "B.Cu") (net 9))
 (segment (start 131.4 71.8) (end 132.6 71.8) (width 0.25) (layer "B.Cu") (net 9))
 (segment (start 132.6 71.8) (end 136.4 68) (width 0.25) (layer "B.Cu") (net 9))
 (segment (start 136.4 66.8) (end 137.17 66.03) (width 0.25) (layer "B.Cu") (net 9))
 (segment (start 136.4 68) (end 136.4 66.8) (width 0.25) (layer "B.Cu") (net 9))
 (segment (start 134.8 71.6) (end 134.175 70.975) (width 0.25) (layer "F.Cu") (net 1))
 (segment (start 127.46 80.24) (end 127.46 82.05) (width 0.25) (layer "F.Cu") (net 1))
 (segment (start 127.25 70.975) (end 127.2 71.025) (width 0.25) (layer "F.Cu") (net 1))
 (segment (start 128.2 79.5) (end 127.46 80.24) (width 0.25) (layer "F.Cu") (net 1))
 (segment (start 124 66) (end 123 66) (width 0.25) (layer "F.Cu") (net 1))
 (segment (start 127.2 71.025) (end 125.625 71.025) (width 0.25) (layer "F.Cu") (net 1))
 (segment (start 131.9 79.5) (end 128.2 79.5) (width 0.25) (layer "F.Cu") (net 1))
 (segment (start 132.54 82.05) (end 133.15 82.05) (width 0.25) (layer "F.Cu") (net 1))
 (segment (start 133.15 82.05) (end 134.2 81) (width 0.25) (layer "F.Cu") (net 1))
 (segment (start 125.275 84.125) (end 126 83.4) (width 0.25) (layer "F.Cu") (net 1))
 (segment (start 126 82.6) (end 126.55 82.05) (width 0.25) (layer "F.Cu") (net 1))
 (segment (start 134.8 73.6) (end 134.8 71.6) (width 0.25) (layer "F.Cu") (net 1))
 (segment (start 125.275 85) (end 125.275 84.125) (width 0.25) (layer "F.Cu") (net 1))
 (segment (start 126 83.4) (end 126 82.6) (width 0.25) (layer "F.Cu") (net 1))
 (segment (start 134.2 81) (end 134.2 74.2) (width 0.25) (layer "F.Cu") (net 1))
 (segment (start 134.2 74.2) (end 134.8 73.6) (width 0.25) (layer "F.Cu") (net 1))
 (segment (start 132.54 82.05) (end 132.54 80.14) (width 0.25) (layer "F.Cu") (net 1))
 (segment (start 124.8 66.8) (end 124 66) (width 0.25) (layer "F.Cu") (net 1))
 (segment (start 125.625 71.025) (end 124.8 70.2) (width 0.25) (layer "F.Cu") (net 1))
 (segment (start 134.175 70.975) (end 133.2 70.975) (width 0.25) (layer "F.Cu") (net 1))
 (segment (start 126.55 82.05) (end 127.46 82.05) (width 0.25) (layer "F.Cu") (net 1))
 (segment (start 132.54 80.14) (end 131.9 79.5) (width 0.25) (layer "F.Cu") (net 1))
 (segment (start 133.2 70.975) (end 127.25 70.975) (width 0.25) (layer "F.Cu") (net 1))
 (segment (start 124.8 70.2) (end 124.8 66.8) (width 0.25) (layer "F.Cu") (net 1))
 (via (at 123 66) (size 0.6) (drill 0.3) (layers "F.Cu" "B.Cu") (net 1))
 (segment (start 123 66) (end 121.14 66) (width 0.25) (layer "B.Cu") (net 1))
 (segment (start 121.14 66) (end 121.11 66.03) (width 0.25) (layer "B.Cu") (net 1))
 (segment (start 131.7 85) (end 132.725 85) (width 0.25) (layer "F.Cu") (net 3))
 (segment (start 131.27 84.57) (end 131.7 85) (width 0.25) (layer "F.Cu") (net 3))
 (segment (start 131.27 82.05) (end 131.27 84.57) (width 0.25) (layer "F.Cu") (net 3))
 (segment (start 127.075 86.45) (end 127.125 86.5) (width 0.25) (layer "F.Cu") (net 4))
 (segment (start 127.075 85) (end 127.075 86.45) (width 0.25) (layer "F.Cu") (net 4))
 (segment (start 128.725 82.055) (end 128.73 82.05) (width 0.3) (layer "F.Cu") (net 5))
 (segment (start 128.725 85) (end 128.725 82.055) (width 0.3) (layer "F.Cu") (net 5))
 (segment (start 121.11 88.89) (end 116.49 88.89) (width 0.25) (layer "B.Cu") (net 13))
 (segment (start 115.8 88.2) (end 115.8 86.8) (width 0.25) (layer "B.Cu") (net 13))
 (segment (start 116.49 88.89) (end 115.8 88.2) (width 0.25) (layer "B.Cu") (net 13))
 (segment (start 114.53 89.93) (end 114.53 86.8) (width 0.25) (layer "B.Cu") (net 14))
 (segment (start 121.11 91.43) (end 116.03 91.43) (width 0.25) (layer "B.Cu") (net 14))
 (segment (start 116.03 91.43) (end 114.53 89.93) (width 0.25) (layer "B.Cu") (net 14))
 (segment (start 114.97 93.97) (end 113.26 92.26) (width 0.25) (layer "B.Cu") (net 15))
 (segment (start 121.11 93.97) (end 114.97 93.97) (width 0.25) (layer "B.Cu") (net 15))
 (segment (start 113.26 92.26) (end 113.26 86.8) (width 0.25) (layer "B.Cu") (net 15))
 (segment (start 114.31 96.51) (end 111.99 94.19) (width 0.25) (layer "B.Cu") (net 16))
 (segment (start 121.11 96.51) (end 114.31 96.51) (width 0.25) (layer "B.Cu") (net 16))
 (segment (start 111.99 94.19) (end 111.99 86.8) (width 0.25) (layer "B.Cu") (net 16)))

